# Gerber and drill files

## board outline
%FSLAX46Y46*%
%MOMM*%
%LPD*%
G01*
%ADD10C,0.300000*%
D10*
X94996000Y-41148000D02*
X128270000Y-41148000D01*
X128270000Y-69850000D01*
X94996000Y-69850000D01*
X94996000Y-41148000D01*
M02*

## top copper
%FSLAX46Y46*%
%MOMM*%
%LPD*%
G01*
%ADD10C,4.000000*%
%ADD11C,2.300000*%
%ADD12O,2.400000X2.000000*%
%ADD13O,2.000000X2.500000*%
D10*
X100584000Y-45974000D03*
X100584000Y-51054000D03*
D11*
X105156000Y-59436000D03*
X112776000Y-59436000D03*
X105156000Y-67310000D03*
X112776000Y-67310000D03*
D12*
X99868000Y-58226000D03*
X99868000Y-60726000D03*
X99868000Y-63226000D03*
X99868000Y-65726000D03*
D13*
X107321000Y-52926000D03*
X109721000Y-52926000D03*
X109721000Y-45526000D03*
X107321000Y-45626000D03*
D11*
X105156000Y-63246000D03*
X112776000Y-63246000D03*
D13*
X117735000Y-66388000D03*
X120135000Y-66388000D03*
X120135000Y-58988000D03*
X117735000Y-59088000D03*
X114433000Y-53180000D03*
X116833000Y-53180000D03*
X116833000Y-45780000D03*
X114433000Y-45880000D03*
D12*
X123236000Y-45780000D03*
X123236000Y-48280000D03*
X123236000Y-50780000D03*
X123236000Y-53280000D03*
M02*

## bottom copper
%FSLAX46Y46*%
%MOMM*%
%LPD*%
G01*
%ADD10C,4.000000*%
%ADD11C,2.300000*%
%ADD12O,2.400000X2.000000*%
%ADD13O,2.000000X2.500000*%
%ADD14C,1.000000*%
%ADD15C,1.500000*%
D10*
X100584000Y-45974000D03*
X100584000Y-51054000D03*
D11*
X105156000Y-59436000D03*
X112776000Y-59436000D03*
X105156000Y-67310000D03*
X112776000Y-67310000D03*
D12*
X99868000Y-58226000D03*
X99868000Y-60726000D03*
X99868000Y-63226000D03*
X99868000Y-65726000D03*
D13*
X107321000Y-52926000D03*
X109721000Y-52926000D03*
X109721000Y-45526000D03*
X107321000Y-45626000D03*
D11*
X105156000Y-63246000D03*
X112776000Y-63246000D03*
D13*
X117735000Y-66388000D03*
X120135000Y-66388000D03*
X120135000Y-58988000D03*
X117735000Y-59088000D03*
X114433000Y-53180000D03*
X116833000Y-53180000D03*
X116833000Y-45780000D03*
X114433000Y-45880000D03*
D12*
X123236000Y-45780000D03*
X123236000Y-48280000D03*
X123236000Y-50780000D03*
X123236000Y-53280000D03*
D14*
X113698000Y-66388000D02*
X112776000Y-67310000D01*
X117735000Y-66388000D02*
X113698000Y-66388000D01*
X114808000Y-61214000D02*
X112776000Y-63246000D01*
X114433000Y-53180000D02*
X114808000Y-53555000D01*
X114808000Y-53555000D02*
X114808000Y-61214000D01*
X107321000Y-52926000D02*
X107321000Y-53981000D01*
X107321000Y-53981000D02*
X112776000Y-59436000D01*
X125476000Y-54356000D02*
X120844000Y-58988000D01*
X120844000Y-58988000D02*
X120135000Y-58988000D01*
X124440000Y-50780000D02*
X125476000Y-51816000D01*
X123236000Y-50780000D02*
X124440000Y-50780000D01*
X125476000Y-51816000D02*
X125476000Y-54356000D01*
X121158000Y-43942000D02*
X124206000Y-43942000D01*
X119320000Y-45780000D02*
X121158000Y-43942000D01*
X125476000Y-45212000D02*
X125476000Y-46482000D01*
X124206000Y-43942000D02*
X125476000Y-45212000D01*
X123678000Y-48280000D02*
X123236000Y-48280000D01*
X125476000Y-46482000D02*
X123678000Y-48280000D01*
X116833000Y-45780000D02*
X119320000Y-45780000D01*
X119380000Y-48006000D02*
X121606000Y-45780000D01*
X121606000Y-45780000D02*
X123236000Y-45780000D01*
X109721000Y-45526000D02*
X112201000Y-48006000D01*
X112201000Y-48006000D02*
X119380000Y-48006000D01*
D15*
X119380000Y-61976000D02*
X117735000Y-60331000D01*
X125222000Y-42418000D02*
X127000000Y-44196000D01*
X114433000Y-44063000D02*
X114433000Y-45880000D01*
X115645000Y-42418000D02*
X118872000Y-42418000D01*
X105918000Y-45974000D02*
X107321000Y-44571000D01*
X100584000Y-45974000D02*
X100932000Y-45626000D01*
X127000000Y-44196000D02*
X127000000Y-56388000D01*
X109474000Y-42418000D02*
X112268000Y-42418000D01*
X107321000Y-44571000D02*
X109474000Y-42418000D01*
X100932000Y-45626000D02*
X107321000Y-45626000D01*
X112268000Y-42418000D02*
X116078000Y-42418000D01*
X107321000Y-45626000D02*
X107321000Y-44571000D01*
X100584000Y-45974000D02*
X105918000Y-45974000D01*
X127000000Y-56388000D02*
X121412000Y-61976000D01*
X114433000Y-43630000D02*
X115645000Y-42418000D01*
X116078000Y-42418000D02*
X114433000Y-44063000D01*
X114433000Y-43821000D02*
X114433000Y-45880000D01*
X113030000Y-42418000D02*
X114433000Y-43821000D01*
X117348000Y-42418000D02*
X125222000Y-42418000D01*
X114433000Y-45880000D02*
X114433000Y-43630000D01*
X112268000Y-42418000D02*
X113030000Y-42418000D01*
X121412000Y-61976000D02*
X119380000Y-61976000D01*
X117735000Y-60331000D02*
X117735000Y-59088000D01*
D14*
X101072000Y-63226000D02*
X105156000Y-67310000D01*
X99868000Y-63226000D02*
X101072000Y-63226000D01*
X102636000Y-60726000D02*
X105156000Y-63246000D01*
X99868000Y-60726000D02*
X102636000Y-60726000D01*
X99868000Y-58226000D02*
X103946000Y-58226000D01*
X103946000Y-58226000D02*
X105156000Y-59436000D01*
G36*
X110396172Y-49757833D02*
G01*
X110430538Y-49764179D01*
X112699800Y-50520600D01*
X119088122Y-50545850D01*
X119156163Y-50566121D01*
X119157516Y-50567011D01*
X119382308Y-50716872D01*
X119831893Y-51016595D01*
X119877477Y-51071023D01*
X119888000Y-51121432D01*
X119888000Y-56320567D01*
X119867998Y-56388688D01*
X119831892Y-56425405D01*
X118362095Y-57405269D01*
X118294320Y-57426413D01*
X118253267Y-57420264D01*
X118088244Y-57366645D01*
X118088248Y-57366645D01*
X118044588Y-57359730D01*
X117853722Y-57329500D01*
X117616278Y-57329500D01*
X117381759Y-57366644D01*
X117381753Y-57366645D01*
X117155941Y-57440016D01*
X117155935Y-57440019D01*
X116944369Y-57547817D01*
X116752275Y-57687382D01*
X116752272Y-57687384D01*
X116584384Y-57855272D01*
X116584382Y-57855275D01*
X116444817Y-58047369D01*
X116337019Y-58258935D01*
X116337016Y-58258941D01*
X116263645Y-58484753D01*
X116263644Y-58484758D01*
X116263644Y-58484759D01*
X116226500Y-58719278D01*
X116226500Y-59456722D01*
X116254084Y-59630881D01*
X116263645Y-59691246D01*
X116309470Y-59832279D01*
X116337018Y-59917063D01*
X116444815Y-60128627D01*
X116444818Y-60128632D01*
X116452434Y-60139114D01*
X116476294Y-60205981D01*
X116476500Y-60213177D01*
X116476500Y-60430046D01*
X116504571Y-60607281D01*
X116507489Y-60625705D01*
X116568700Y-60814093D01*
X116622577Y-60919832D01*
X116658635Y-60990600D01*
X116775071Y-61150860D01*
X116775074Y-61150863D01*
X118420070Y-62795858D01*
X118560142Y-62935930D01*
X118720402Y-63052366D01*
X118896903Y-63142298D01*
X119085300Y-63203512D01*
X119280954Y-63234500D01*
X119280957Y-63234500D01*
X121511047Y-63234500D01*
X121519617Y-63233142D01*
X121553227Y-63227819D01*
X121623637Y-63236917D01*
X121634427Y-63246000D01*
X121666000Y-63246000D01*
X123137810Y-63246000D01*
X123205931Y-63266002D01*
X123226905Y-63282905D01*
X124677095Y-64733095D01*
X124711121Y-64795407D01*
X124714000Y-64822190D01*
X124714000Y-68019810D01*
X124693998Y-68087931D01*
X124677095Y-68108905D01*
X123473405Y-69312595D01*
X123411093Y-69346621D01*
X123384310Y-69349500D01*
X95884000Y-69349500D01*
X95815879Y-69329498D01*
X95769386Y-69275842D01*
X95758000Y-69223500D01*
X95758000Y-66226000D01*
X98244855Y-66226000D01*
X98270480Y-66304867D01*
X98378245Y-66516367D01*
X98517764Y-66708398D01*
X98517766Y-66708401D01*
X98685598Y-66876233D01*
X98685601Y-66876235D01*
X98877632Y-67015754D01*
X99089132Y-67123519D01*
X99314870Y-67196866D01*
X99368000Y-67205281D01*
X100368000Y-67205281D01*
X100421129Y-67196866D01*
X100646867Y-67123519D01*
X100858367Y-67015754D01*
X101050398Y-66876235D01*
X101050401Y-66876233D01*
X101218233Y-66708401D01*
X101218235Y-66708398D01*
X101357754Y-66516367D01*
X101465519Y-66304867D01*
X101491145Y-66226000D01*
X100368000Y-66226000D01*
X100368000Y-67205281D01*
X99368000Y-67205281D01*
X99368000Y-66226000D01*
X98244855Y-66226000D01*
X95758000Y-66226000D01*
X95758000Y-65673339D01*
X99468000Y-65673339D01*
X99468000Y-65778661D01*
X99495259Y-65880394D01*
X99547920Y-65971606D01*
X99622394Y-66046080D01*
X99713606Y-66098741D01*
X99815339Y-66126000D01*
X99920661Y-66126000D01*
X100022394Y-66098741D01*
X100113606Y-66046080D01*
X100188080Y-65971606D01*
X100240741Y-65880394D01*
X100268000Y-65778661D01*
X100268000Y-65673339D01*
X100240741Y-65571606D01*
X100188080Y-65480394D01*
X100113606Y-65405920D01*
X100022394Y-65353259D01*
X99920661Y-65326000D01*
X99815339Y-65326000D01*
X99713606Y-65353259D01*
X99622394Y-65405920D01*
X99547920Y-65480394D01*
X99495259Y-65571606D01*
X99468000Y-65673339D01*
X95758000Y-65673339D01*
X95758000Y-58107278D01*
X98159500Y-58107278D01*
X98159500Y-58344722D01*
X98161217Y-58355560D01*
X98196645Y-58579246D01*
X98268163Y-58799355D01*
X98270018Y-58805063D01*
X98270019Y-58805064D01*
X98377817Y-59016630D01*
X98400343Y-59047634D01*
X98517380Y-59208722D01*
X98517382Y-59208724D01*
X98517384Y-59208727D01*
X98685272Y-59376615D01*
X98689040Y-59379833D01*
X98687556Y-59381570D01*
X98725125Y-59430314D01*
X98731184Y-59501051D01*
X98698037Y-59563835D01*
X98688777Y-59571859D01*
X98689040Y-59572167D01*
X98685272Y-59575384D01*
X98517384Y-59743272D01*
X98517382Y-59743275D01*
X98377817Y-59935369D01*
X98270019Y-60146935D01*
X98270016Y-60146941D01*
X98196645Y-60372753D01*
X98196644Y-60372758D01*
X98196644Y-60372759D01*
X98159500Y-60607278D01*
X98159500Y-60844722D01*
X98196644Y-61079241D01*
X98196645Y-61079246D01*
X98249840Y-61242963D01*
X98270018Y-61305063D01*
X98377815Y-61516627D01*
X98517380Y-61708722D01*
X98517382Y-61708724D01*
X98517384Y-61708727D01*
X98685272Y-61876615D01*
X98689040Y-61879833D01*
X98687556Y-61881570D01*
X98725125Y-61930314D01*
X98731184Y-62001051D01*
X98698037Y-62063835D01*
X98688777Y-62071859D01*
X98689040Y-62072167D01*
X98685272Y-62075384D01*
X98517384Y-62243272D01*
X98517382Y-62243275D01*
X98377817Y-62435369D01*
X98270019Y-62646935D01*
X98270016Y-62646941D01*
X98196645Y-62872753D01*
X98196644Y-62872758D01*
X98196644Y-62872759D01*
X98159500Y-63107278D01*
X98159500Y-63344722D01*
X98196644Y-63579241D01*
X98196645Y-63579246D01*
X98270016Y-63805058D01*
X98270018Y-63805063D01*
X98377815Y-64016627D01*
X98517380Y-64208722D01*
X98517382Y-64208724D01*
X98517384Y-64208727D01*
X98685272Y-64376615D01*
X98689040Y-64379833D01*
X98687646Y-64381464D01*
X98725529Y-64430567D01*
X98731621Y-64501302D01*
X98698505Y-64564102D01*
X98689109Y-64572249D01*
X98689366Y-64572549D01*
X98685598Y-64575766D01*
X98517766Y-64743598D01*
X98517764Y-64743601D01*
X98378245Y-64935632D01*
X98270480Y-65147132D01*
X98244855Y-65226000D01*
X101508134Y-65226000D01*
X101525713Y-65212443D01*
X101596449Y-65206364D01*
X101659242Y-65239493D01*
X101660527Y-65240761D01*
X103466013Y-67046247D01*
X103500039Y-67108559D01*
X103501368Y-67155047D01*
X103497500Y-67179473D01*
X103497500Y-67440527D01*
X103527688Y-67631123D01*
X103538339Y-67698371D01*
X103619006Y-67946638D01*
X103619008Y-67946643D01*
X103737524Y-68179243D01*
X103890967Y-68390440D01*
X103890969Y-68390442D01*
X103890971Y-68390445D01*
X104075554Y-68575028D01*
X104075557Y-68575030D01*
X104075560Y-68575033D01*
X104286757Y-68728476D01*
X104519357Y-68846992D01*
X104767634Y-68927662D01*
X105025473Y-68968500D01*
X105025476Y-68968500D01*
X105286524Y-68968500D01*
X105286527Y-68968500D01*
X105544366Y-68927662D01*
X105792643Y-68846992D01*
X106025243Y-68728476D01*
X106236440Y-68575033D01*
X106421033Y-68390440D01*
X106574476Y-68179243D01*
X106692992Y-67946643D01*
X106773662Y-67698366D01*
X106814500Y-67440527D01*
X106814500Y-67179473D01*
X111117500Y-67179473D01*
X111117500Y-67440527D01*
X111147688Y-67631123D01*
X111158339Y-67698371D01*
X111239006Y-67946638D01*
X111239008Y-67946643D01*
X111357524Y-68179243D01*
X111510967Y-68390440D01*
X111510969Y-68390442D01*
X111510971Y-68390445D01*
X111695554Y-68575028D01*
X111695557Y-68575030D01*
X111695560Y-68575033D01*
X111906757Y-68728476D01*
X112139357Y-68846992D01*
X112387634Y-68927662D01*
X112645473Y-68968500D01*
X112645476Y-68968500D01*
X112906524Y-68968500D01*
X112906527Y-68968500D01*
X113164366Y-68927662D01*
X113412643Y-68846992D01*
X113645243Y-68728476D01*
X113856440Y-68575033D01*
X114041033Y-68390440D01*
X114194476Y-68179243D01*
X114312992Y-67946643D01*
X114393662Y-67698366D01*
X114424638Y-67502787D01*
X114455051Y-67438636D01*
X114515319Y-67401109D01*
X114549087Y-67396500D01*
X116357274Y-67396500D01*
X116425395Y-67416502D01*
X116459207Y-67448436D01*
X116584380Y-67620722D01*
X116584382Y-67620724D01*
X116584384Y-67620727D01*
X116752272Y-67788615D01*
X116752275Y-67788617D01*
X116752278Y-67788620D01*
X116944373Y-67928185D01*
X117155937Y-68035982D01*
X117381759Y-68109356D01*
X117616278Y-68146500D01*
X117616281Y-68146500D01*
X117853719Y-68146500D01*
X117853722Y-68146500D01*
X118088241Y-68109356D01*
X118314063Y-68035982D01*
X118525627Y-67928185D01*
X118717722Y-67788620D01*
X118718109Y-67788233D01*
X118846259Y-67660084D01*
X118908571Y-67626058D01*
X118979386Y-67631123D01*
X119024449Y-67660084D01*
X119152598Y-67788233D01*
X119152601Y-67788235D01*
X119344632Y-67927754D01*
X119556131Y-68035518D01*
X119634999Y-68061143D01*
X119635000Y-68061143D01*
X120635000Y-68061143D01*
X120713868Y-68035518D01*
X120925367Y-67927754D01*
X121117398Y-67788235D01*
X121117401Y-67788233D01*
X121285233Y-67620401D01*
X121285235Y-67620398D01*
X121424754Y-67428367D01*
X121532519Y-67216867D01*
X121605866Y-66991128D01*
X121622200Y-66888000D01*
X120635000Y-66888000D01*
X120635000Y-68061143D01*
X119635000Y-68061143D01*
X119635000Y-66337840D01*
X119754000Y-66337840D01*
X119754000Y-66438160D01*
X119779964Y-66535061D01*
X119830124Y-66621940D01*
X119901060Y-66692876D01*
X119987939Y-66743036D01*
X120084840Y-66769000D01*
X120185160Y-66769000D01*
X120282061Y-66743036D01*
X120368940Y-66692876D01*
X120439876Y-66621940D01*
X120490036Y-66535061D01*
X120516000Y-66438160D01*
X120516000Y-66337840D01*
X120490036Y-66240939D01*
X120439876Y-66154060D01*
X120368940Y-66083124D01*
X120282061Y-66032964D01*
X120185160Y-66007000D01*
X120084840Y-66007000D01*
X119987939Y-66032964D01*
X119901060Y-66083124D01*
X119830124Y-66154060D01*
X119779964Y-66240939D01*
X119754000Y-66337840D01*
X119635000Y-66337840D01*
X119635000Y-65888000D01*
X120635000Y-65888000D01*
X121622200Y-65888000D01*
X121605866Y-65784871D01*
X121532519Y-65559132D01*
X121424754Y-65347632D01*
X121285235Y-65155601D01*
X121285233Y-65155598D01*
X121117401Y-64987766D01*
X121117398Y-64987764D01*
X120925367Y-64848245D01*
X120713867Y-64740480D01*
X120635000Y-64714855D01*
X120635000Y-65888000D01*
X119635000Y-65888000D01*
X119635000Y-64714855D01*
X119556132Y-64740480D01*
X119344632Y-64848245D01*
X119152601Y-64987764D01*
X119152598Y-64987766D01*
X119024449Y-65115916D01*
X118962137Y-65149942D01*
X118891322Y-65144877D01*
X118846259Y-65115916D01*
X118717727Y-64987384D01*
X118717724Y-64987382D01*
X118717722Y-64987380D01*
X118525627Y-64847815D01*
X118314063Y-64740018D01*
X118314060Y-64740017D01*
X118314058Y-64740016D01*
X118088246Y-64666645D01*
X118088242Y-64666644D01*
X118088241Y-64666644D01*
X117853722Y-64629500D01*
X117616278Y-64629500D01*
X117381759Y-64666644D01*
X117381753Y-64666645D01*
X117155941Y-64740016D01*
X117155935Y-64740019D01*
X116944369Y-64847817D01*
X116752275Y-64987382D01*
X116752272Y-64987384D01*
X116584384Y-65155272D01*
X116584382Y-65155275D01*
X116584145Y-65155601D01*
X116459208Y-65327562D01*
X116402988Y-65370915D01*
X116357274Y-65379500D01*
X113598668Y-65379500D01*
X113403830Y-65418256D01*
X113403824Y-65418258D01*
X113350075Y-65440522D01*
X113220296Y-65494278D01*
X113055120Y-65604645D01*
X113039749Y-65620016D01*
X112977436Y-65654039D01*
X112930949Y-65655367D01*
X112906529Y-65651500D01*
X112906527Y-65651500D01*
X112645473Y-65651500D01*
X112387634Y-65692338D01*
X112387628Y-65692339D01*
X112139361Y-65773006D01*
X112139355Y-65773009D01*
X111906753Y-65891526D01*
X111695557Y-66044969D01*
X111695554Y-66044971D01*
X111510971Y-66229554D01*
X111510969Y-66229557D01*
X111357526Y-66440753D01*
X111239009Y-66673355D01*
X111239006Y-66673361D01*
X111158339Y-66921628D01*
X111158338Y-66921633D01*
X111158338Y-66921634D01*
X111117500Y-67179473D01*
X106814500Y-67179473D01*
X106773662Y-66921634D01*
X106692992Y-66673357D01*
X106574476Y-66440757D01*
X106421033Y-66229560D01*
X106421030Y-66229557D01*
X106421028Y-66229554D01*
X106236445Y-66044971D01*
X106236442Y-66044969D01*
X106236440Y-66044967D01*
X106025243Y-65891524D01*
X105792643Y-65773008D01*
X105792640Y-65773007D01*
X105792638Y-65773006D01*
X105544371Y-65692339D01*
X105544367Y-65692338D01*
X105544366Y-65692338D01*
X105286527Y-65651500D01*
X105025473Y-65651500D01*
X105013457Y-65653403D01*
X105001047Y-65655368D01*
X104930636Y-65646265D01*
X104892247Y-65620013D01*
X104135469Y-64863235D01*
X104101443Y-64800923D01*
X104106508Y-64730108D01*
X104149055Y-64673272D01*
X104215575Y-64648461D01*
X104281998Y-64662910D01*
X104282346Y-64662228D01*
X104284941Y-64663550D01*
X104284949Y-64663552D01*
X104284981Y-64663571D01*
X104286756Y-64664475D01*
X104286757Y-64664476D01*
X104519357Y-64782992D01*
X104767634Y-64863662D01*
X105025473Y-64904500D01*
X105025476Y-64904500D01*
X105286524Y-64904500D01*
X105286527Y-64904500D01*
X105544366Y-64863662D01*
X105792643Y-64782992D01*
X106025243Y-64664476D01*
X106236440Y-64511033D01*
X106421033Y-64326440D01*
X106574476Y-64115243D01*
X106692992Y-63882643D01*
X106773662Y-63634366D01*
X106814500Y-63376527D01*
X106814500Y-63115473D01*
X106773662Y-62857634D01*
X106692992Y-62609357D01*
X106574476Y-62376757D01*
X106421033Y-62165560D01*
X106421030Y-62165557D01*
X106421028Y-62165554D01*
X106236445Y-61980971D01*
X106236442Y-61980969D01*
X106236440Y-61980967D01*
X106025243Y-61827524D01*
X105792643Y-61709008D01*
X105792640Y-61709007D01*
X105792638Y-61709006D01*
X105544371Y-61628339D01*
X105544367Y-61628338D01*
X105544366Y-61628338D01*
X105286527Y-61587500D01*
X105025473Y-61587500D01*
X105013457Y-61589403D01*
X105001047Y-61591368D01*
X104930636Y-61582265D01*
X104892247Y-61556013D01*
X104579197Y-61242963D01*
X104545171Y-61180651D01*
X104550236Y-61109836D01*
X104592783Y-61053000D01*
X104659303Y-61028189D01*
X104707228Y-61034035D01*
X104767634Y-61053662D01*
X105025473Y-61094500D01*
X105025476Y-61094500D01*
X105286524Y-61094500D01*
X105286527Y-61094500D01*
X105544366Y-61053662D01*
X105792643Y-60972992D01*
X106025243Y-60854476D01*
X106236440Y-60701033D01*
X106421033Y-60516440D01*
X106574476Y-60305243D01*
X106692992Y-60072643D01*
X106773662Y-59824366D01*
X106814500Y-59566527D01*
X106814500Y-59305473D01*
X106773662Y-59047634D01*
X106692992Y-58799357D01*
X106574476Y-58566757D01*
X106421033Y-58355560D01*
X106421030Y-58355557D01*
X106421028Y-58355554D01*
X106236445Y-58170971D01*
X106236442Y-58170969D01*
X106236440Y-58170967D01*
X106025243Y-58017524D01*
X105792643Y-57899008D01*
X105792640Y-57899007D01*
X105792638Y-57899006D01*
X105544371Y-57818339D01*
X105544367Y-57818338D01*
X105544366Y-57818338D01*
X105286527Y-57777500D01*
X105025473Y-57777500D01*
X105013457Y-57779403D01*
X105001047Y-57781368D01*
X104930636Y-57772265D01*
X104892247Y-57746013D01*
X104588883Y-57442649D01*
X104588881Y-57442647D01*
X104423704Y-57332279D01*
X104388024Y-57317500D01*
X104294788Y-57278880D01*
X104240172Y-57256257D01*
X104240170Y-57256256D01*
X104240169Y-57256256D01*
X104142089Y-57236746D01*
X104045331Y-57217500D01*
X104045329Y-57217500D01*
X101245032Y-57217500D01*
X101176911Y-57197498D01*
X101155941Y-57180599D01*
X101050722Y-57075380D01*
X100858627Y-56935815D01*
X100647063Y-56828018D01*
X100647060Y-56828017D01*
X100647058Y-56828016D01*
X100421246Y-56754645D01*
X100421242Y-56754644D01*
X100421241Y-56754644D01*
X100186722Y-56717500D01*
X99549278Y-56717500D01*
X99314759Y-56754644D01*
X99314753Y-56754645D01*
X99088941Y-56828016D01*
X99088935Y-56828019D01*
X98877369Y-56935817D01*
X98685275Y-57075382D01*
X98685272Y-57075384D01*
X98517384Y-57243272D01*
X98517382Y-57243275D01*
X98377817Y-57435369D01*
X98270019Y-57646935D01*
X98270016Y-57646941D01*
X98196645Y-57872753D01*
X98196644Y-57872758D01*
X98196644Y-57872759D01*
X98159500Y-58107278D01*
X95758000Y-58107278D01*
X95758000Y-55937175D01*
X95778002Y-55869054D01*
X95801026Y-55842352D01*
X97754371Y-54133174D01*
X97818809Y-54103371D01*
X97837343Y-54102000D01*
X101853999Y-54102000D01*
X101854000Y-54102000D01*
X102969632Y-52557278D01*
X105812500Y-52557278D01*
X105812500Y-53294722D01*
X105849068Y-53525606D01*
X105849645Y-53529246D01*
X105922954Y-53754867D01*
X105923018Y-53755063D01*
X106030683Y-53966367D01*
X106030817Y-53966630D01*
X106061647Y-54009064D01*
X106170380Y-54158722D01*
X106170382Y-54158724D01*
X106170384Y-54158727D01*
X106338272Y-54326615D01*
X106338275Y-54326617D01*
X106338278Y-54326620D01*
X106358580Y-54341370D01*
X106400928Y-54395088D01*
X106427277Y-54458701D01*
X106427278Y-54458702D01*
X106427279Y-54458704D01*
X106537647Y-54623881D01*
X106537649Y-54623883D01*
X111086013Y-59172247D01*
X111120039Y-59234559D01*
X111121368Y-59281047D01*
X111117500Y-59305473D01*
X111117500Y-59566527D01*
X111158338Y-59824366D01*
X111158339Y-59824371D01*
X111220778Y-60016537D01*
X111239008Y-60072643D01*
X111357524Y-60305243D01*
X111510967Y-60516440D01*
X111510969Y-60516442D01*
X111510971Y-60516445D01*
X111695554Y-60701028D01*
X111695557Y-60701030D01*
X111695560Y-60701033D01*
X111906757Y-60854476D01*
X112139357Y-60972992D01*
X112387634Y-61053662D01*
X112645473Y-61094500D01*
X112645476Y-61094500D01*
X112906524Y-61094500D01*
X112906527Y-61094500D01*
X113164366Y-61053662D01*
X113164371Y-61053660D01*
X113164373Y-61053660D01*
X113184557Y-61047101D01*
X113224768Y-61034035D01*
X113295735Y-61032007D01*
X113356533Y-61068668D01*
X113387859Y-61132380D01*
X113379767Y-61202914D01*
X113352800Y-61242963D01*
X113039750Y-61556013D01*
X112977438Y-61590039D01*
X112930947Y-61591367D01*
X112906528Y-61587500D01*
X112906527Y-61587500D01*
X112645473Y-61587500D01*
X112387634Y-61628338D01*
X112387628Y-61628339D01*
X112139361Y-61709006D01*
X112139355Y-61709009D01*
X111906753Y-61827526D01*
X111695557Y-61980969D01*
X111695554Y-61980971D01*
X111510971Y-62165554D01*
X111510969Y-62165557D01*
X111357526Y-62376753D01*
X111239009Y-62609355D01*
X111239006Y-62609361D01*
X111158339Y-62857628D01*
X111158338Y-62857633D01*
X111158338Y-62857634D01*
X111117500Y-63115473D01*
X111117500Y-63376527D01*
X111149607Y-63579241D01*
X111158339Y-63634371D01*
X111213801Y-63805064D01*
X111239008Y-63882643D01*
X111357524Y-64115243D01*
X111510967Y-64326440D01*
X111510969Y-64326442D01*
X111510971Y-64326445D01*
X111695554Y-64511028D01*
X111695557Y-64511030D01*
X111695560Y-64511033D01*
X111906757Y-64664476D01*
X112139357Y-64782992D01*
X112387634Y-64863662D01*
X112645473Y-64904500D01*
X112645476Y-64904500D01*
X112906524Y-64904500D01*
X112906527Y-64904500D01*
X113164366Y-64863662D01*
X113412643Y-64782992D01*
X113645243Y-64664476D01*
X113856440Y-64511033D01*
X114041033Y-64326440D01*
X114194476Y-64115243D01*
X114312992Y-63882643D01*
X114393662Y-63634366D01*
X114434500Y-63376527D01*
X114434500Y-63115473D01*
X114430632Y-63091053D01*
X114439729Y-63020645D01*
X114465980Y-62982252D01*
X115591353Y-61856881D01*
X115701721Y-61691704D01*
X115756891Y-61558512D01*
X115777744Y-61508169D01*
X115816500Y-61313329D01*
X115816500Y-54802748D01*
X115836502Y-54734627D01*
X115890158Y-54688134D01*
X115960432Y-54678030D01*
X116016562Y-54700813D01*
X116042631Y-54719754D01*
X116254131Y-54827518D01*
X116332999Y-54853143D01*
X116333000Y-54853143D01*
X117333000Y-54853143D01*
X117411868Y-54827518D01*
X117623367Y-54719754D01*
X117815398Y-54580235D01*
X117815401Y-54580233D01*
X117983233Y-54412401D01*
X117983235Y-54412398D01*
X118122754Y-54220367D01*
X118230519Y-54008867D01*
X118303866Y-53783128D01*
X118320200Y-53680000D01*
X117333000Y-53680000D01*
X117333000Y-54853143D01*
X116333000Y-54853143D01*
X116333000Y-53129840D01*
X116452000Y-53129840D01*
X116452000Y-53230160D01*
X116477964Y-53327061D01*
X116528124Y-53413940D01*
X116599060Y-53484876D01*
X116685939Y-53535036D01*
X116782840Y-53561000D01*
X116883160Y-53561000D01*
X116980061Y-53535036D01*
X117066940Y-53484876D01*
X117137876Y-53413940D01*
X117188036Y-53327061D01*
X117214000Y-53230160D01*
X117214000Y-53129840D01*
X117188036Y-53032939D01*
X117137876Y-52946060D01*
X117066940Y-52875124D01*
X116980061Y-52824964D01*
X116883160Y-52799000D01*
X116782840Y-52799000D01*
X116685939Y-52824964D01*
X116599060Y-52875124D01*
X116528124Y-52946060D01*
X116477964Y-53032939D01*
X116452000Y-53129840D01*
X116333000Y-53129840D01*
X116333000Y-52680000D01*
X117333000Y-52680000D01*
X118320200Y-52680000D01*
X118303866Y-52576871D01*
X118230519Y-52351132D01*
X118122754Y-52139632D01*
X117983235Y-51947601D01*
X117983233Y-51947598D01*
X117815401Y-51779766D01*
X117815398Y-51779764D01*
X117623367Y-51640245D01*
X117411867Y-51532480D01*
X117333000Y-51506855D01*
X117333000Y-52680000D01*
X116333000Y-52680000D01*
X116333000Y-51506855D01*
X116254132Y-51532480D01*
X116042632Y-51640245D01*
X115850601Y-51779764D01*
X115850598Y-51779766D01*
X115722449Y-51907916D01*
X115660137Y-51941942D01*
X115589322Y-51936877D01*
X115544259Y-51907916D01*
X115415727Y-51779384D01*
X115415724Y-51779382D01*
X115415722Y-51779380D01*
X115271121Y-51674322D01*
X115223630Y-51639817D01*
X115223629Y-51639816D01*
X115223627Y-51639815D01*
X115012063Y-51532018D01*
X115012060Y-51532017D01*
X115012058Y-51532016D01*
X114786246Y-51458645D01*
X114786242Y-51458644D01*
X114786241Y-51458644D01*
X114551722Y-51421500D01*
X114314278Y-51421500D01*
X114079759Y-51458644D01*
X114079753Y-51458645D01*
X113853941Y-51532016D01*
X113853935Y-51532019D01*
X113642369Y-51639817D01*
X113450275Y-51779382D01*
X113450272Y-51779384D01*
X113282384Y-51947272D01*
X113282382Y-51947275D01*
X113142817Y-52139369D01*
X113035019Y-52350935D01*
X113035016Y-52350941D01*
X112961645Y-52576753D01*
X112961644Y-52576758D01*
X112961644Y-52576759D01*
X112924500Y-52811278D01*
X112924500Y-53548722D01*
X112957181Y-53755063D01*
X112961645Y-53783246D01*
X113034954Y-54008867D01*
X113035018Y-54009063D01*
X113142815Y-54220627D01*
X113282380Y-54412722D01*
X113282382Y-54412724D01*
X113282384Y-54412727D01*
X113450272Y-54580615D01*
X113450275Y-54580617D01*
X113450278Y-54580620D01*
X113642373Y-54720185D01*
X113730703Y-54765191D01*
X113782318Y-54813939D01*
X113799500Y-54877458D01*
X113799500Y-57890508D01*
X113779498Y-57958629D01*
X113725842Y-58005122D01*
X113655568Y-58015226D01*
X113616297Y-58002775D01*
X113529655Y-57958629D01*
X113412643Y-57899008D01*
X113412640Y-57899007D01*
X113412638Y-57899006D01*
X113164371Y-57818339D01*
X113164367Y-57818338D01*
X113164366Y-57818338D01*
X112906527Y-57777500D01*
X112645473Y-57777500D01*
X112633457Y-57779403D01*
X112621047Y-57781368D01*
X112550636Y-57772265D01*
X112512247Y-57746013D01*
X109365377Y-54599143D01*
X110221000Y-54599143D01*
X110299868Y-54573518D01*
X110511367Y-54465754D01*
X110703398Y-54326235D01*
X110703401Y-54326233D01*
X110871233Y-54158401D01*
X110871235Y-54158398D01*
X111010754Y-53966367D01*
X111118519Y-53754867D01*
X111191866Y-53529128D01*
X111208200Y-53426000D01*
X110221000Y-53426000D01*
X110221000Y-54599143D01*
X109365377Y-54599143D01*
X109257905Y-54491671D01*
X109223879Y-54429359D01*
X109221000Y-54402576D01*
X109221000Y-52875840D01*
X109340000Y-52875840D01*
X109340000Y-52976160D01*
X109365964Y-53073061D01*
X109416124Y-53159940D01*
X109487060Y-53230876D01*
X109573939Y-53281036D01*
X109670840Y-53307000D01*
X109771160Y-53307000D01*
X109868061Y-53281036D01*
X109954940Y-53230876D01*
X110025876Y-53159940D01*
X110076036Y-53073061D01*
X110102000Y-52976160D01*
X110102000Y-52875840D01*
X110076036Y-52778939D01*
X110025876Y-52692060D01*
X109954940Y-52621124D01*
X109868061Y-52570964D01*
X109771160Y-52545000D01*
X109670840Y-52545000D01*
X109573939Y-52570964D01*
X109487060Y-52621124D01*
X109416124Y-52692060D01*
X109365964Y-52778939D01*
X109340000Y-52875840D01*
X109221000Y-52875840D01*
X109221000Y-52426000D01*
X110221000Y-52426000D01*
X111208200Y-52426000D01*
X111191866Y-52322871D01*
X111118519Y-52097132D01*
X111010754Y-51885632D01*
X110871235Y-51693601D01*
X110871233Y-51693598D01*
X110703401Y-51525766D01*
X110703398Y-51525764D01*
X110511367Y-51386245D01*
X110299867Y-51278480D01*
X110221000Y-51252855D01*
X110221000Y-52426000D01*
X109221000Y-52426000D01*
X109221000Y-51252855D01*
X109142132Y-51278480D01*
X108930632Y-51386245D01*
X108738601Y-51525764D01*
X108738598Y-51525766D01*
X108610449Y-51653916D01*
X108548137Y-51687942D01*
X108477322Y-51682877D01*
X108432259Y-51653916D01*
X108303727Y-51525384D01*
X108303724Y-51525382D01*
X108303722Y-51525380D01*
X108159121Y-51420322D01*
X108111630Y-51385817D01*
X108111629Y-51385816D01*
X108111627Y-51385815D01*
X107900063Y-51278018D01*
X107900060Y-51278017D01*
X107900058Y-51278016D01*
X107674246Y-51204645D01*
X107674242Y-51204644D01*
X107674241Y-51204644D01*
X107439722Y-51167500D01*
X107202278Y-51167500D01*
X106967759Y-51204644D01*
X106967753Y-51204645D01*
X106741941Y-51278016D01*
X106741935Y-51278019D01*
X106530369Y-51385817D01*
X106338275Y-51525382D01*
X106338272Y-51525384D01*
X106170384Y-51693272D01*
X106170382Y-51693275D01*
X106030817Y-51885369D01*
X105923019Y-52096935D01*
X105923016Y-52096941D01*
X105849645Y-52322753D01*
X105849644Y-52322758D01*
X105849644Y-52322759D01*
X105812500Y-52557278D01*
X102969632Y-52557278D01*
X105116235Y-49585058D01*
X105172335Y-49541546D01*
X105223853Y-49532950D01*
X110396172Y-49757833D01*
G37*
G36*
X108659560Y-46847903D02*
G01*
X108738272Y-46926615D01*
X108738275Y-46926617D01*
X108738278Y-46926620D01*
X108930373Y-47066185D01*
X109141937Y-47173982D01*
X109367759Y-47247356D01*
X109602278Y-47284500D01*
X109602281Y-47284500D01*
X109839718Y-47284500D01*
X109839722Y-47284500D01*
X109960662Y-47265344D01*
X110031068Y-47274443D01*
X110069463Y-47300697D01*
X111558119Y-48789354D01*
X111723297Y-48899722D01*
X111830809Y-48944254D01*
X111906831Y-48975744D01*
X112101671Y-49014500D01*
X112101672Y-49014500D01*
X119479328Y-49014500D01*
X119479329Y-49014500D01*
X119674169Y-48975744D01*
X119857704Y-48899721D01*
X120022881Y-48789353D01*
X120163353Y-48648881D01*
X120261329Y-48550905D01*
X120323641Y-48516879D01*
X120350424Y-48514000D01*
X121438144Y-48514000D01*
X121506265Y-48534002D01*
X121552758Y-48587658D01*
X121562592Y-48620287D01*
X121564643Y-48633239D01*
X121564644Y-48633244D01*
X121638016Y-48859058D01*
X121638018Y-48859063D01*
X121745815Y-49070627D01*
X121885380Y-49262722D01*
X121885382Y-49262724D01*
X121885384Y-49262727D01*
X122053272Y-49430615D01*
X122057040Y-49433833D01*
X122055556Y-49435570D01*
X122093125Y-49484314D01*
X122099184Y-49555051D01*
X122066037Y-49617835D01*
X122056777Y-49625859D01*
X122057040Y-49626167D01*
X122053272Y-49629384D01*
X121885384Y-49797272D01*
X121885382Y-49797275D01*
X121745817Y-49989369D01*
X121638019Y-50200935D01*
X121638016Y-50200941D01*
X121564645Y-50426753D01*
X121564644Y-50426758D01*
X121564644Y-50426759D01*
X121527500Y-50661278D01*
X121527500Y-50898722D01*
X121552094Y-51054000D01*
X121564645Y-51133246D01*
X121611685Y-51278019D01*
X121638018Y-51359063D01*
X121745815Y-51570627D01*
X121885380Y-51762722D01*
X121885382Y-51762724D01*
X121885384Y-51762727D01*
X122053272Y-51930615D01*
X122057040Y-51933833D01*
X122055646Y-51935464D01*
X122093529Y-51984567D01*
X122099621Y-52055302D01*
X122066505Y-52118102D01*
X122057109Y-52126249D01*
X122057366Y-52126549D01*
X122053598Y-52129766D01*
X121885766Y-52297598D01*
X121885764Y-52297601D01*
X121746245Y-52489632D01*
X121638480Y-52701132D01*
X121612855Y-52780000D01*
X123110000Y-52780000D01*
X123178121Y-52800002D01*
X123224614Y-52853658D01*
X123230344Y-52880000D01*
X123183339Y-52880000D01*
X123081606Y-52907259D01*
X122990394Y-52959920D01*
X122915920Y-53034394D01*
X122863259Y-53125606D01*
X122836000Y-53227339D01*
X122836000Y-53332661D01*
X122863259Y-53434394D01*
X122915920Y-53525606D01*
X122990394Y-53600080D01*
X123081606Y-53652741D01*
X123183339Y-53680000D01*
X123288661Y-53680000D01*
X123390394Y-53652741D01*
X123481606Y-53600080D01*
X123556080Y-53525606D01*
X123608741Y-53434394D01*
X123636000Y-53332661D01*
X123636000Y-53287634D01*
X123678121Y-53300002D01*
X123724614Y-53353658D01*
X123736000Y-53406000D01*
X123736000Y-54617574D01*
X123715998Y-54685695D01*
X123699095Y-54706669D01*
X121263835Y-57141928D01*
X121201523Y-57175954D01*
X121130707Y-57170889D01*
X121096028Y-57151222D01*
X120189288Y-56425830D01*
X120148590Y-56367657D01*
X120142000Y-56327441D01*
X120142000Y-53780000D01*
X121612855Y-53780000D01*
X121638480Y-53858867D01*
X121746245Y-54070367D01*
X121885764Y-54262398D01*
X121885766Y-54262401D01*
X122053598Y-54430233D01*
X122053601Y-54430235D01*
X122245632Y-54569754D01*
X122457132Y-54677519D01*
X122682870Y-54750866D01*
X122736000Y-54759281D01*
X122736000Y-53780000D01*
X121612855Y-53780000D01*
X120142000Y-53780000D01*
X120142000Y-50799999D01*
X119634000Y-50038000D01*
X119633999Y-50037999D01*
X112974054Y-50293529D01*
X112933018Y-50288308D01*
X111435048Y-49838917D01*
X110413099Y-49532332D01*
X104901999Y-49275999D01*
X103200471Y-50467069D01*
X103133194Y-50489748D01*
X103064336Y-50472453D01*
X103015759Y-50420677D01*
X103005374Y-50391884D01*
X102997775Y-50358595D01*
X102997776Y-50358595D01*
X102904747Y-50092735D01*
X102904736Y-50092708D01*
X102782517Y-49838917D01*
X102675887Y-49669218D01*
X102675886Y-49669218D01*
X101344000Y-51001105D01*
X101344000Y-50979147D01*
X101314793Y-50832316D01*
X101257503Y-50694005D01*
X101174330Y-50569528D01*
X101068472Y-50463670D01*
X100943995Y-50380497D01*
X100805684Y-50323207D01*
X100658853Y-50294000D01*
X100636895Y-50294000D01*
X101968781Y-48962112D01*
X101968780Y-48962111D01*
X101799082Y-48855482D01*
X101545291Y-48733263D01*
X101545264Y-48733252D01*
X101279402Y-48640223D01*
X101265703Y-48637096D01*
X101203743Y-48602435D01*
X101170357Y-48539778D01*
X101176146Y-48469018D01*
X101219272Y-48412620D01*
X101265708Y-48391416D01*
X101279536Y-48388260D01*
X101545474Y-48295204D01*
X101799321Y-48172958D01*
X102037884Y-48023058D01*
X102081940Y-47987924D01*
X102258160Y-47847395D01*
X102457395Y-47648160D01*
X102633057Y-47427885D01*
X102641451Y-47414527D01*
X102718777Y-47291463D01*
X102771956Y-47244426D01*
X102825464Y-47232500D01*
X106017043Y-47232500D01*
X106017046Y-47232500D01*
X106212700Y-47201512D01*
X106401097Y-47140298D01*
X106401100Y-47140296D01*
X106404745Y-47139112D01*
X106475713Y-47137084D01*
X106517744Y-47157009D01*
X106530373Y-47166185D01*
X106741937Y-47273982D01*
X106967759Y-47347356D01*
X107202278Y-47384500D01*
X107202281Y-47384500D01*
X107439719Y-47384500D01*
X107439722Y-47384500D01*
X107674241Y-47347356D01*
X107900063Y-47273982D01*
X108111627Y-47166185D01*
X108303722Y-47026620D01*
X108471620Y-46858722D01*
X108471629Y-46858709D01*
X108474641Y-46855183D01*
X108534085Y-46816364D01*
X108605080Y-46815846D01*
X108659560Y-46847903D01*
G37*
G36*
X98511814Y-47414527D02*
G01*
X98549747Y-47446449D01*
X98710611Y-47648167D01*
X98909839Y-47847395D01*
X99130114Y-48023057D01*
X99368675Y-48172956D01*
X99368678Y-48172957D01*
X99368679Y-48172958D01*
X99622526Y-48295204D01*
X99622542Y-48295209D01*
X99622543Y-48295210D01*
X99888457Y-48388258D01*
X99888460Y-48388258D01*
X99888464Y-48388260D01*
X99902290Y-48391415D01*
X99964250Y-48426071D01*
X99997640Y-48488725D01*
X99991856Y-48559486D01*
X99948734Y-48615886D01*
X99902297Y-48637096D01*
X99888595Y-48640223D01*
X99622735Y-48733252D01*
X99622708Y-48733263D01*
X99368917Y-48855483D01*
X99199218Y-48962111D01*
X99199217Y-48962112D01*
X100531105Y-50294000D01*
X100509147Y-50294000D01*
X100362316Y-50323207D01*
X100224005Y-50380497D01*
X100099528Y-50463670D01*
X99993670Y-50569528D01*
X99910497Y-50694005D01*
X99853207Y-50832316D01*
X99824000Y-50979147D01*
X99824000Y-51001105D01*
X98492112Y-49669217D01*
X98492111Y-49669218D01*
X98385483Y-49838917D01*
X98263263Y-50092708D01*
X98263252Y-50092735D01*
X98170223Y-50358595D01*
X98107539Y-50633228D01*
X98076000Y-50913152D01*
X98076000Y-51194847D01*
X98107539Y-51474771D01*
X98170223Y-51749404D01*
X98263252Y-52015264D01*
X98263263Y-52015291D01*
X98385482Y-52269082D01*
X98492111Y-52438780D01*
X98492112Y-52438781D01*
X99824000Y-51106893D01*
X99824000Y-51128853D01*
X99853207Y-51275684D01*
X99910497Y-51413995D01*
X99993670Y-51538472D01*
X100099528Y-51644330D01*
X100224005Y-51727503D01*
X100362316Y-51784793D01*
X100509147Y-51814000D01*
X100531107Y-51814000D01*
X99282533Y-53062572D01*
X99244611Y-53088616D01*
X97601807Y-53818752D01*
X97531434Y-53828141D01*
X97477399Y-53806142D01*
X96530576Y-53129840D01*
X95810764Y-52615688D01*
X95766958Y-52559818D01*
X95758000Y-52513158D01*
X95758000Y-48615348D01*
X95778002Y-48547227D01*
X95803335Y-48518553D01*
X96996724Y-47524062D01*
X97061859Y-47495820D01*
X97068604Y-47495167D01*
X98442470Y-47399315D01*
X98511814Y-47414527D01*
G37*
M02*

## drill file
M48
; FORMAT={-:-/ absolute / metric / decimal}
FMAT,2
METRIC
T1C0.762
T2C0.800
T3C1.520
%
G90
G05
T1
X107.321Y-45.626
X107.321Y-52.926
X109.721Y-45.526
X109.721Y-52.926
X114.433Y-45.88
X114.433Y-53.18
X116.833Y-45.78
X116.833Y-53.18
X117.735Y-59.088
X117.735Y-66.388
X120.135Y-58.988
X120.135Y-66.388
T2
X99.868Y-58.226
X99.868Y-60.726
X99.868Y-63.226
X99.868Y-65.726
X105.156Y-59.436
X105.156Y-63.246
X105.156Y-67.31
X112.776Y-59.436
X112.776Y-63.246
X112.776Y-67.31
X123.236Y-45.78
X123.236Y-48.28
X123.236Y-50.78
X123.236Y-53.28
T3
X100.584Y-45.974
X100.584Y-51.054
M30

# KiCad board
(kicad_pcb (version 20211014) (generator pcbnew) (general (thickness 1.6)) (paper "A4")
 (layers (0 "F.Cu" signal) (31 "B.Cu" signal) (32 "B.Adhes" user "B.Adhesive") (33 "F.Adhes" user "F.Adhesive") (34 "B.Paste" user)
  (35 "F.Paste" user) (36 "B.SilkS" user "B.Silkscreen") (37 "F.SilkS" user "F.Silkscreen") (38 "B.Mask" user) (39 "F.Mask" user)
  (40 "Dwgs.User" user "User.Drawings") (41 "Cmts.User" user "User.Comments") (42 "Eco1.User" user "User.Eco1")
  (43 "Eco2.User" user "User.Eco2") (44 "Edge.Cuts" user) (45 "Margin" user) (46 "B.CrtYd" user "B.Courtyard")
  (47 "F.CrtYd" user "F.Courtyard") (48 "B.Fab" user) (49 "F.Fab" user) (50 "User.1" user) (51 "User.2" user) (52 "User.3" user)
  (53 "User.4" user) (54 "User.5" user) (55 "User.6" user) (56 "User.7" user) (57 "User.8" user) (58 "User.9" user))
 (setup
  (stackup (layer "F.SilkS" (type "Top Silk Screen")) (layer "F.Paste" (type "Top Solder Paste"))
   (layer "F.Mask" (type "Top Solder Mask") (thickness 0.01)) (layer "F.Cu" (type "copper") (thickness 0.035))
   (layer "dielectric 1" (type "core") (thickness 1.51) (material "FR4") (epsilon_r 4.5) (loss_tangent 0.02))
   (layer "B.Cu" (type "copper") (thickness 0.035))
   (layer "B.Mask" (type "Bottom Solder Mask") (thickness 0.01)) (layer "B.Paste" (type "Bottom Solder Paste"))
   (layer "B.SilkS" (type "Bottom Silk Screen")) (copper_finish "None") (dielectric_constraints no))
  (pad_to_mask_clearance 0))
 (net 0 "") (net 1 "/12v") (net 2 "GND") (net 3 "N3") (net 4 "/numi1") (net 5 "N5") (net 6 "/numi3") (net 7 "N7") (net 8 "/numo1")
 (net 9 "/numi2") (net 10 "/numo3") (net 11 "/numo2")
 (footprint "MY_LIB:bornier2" (layer "F.Cu") (at 100.584 45.974 -90)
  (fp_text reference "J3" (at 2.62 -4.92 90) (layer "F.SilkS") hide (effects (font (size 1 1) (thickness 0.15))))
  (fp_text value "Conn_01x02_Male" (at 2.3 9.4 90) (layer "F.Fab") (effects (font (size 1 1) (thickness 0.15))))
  (pad "1" thru_hole circle locked (at 0 0 270) (size 4 4) (drill 1.52) (layers *.Cu *.Mask) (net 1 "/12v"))
  (pad "2" thru_hole circle locked (at 5.08 0 270) (size 4 4) (drill 1.52) (layers *.Cu *.Mask) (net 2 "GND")))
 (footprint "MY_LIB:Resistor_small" (layer "F.Cu") (at 105.156 59.436)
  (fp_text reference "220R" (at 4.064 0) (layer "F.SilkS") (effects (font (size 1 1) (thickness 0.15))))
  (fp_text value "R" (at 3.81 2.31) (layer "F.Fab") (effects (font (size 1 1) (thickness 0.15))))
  (pad "1" thru_hole circle locked (at 0 0) (size 2.3 2.3) (drill 0.8) (layers *.Cu *.Mask) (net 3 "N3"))
  (pad "2" thru_hole circle locked (at 7.62 0) (size 2.3 2.3) (drill 0.8) (layers *.Cu *.Mask) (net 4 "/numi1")))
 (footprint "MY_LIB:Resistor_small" (layer "F.Cu") (at 105.156 67.31)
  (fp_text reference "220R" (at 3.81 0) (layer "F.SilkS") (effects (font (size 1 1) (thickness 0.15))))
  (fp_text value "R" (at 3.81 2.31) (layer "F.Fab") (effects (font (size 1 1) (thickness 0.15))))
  (pad "1" thru_hole circle locked (at 0 0) (size 2.3 2.3) (drill 0.8) (layers *.Cu *.Mask) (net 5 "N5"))
  (pad "2" thru_hole circle locked (at 7.62 0) (size 2.3 2.3) (drill 0.8) (layers *.Cu *.Mask) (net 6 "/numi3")))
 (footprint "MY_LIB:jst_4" (layer "F.Cu") (at 99.868 58.226 -90)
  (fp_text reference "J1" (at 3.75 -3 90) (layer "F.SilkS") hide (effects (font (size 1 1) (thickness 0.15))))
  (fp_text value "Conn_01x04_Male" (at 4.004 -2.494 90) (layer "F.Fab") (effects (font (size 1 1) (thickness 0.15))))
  (pad "1" thru_hole oval locked (at 0 0 270) (size 2 2.4) (drill 0.8) (layers *.Cu *.Mask) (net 3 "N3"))
  (pad "2" thru_hole oval locked (at 2.5 0 270) (size 2 2.4) (drill 0.8) (layers *.Cu *.Mask) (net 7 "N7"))
  (pad "3" thru_hole oval locked (at 5 0 270) (size 2 2.4) (drill 0.8) (layers *.Cu *.Mask) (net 5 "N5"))
  (pad "4" thru_hole oval locked (at 7.5 0 270) (size 2 2.4) (drill 0.8) (layers *.Cu *.Mask) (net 2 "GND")))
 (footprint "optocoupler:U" (layer "F.Cu") (at 112.121 50.026 90)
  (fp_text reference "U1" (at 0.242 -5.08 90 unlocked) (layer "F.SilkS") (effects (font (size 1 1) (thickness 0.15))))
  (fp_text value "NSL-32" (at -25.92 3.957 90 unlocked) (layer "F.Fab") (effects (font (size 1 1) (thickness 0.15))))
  (pad "1" thru_hole oval (at -2.9 -4.8 90) (size 2.5 2) (drill 0.762) (layers *.Cu *.Mask) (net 4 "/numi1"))
  (pad "2" thru_hole oval (at -2.9 -2.4 90) (size 2.5 2) (drill 0.762) (layers *.Cu *.Mask) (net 2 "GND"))
  (pad "3" thru_hole oval (at 4.5 -2.4 90) (size 2.5 2) (drill 0.762) (layers *.Cu *.Mask) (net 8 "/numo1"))
  (pad "4" thru_hole oval (at 4.4 -4.8 90) (size 2.5 2) (drill 0.762) (layers *.Cu *.Mask) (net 1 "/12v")))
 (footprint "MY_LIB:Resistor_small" (layer "F.Cu") (at 105.156 63.246)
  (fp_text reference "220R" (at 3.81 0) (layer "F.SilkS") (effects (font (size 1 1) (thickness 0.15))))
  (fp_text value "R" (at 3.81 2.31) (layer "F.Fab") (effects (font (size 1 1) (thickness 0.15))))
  (pad "1" thru_hole circle locked (at 0 0) (size 2.3 2.3) (drill 0.8) (layers *.Cu *.Mask) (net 7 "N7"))
  (pad "2" thru_hole circle locked (at 7.62 0) (size 2.3 2.3) (drill 0.8) (layers *.Cu *.Mask) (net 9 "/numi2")))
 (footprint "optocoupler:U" (layer "F.Cu") (at 122.535 63.488 90)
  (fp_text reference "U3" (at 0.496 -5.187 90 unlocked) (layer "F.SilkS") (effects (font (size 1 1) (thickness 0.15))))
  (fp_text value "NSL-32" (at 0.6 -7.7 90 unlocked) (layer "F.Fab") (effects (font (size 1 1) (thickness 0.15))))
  (pad "1" thru_hole oval (at -2.9 -4.8 90) (size 2.5 2) (drill 0.762) (layers *.Cu *.Mask) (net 6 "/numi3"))
  (pad "2" thru_hole oval (at -2.9 -2.4 90) (size 2.5 2) (drill 0.762) (layers *.Cu *.Mask) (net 2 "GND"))
  (pad "3" thru_hole oval (at 4.5 -2.4 90) (size 2.5 2) (drill 0.762) (layers *.Cu *.Mask) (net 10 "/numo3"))
  (pad "4" thru_hole oval (at 4.4 -4.8 90) (size 2.5 2) (drill 0.762) (layers *.Cu *.Mask) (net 1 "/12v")))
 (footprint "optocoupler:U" (layer "F.Cu") (at 119.233 50.28 90)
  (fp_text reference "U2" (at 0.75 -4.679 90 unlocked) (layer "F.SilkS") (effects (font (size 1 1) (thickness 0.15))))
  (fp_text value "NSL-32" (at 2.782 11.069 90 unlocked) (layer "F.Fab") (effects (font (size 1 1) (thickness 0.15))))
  (pad "1" thru_hole oval (at -2.9 -4.8 90) (size 2.5 2) (drill 0.762) (layers *.Cu *.Mask) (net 9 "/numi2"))
  (pad "2" thru_hole oval (at -2.9 -2.4 90) (size 2.5 2) (drill 0.762) (layers *.Cu *.Mask) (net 2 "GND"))
  (pad "3" thru_hole oval (at 4.5 -2.4 90) (size 2.5 2) (drill 0.762) (layers *.Cu *.Mask) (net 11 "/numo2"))
  (pad "4" thru_hole oval (at 4.4 -4.8 90) (size 2.5 2) (drill 0.762) (layers *.Cu *.Mask) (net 1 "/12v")))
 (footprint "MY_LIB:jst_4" (layer "F.Cu") (at 123.236 45.78 -90)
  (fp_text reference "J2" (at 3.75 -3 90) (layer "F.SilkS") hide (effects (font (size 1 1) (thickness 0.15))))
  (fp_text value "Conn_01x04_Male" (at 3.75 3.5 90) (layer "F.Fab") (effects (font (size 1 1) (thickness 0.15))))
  (pad "1" thru_hole oval locked (at 0 0 270) (size 2 2.4) (drill 0.8) (layers *.Cu *.Mask) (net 8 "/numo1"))
  (pad "2" thru_hole oval locked (at 2.5 0 270) (size 2 2.4) (drill 0.8) (layers *.Cu *.Mask) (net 11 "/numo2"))
  (pad "3" thru_hole oval locked (at 5 0 270) (size 2 2.4) (drill 0.8) (layers *.Cu *.Mask) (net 10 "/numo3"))
  (pad "4" thru_hole oval locked (at 7.5 0 270) (size 2 2.4) (drill 0.8) (layers *.Cu *.Mask) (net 2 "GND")))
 (gr_rect (start 94.996 41.148) (end 128.27 69.85) (layer "Edge.Cuts") (width 0.3) (fill none))
 (segment (start 113.698 66.388) (end 112.776 67.31) (width 1) (layer "B.Cu") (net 6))
 (segment (start 117.735 66.388) (end 113.698 66.388) (width 1) (layer "B.Cu") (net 6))
 (segment (start 114.808 61.214) (end 112.776 63.246) (width 1) (layer "B.Cu") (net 9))
 (segment (start 114.433 53.18) (end 114.808 53.555) (width 1) (layer "B.Cu") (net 9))
 (segment (start 114.808 53.555) (end 114.808 61.214) (width 1) (layer "B.Cu") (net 9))
 (segment (start 107.321 52.926) (end 107.321 53.981) (width 1) (layer "B.Cu") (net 4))
 (segment (start 107.321 53.981) (end 112.776 59.436) (width 1) (layer "B.Cu") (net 4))
 (segment (start 125.476 54.356) (end 120.844 58.988) (width 1) (layer "B.Cu") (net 10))
 (segment (start 120.844 58.988) (end 120.135 58.988) (width 1) (layer "B.Cu") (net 10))
 (segment (start 124.44 50.78) (end 125.476 51.816) (width 1) (layer "B.Cu") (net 10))
 (segment (start 123.236 50.78) (end 124.44 50.78) (width 1) (layer "B.Cu") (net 10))
 (segment (start 125.476 51.816) (end 125.476 54.356) (width 1) (layer "B.Cu") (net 10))
 (segment (start 121.158 43.942) (end 124.206 43.942) (width 1) (layer "B.Cu") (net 11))
 (segment (start 119.32 45.78) (end 121.158 43.942) (width 1) (layer "B.Cu") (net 11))
 (segment (start 125.476 45.212) (end 125.476 46.482) (width 1) (layer "B.Cu") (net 11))
 (segment (start 124.206 43.942) (end 125.476 45.212) (width 1) (layer "B.Cu") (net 11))
 (segment (start 123.678 48.28) (end 123.236 48.28) (width 1) (layer "B.Cu") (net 11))
 (segment (start 125.476 46.482) (end 123.678 48.28) (width 1) (layer "B.Cu") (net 11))
 (segment (start 116.833 45.78) (end 119.32 45.78) (width 1) (layer "B.Cu") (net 11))
 (segment (start 119.38 48.006) (end 121.606 45.78) (width 1) (layer "B.Cu") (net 8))
 (segment (start 121.606 45.78) (end 123.236 45.78) (width 1) (layer "B.Cu") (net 8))
 (segment (start 109.721 45.526) (end 112.201 48.006) (width 1) (layer "B.Cu") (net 8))
 (segment (start 112.201 48.006) (end 119.38 48.006) (width 1) (layer "B.Cu") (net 8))
 (segment (start 119.38 61.976) (end 117.735 60.331) (width 1.5) (layer "B.Cu") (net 1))
 (segment (start 125.222 42.418) (end 127 44.196) (width 1.5) (layer "B.Cu") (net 1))
 (segment (start 114.433 44.063) (end 114.433 45.88) (width 1.5) (layer "B.Cu") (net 1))
 (segment (start 115.645 42.418) (end 118.872 42.418) (width 1.5) (layer "B.Cu") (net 1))
 (segment (start 105.918 45.974) (end 107.321 44.571) (width 1.5) (layer "B.Cu") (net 1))
 (segment (start 100.584 45.974) (end 100.932 45.626) (width 1.5) (layer "B.Cu") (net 1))
 (segment (start 127 44.196) (end 127 56.388) (width 1.5) (layer "B.Cu") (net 1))
 (segment (start 109.474 42.418) (end 112.268 42.418) (width 1.5) (layer "B.Cu") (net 1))
 (segment (start 107.321 44.571) (end 109.474 42.418) (width 1.5) (layer "B.Cu") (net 1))
 (segment (start 100.932 45.626) (end 107.321 45.626) (width 1.5) (layer "B.Cu") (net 1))
 (segment (start 112.268 42.418) (end 116.078 42.418) (width 1.5) (layer "B.Cu") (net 1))
 (segment (start 107.321 45.626) (end 107.321 44.571) (width 1.5) (layer "B.Cu") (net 1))
 (segment (start 100.584 45.974) (end 105.918 45.974) (width 1.5) (layer "B.Cu") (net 1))
 (segment (start 127 56.388) (end 121.412 61.976) (width 1.5) (layer "B.Cu") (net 1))
 (segment (start 114.433 43.63) (end 115.645 42.418) (width 1.5) (layer "B.Cu") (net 1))
 (segment (start 116.078 42.418) (end 114.433 44.063) (width 1.5) (layer "B.Cu") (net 1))
 (segment (start 114.433 43.821) (end 114.433 45.88) (width 1.5) (layer "B.Cu") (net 1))
 (segment (start 113.03 42.418) (end 114.433 43.821) (width 1.5) (layer "B.Cu") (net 1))
 (segment (start 117.348 42.418) (end 125.222 42.418) (width 1.5) (layer "B.Cu") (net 1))
 (segment (start 114.433 45.88) (end 114.433 43.63) (width 1.5) (layer "B.Cu") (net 1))
 (segment (start 112.268 42.418) (end 113.03 42.418) (width 1.5) (layer "B.Cu") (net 1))
 (segment (start 121.412 61.976) (end 119.38 61.976) (width 1.5) (layer "B.Cu") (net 1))
 (segment (start 117.735 60.331) (end 117.735 59.088) (width 1.5) (layer "B.Cu") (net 1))
 (segment (start 101.072 63.226) (end 105.156 67.31) (width 1) (layer "B.Cu") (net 5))
 (segment (start 99.868 63.226) (end 101.072 63.226) (width 1) (layer "B.Cu") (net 5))
 (segment (start 102.636 60.726) (end 105.156 63.246) (width 1) (layer "B.Cu") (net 7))
 (segment (start 99.868 60.726) (end 102.636 60.726) (width 1) (layer "B.Cu") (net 7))
 (segment (start 99.868 58.226) (end 103.946 58.226) (width 1) (layer "B.Cu") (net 3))
 (segment (start 103.946 58.226) (end 105.156 59.436) (width 1) (layer "B.Cu") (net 3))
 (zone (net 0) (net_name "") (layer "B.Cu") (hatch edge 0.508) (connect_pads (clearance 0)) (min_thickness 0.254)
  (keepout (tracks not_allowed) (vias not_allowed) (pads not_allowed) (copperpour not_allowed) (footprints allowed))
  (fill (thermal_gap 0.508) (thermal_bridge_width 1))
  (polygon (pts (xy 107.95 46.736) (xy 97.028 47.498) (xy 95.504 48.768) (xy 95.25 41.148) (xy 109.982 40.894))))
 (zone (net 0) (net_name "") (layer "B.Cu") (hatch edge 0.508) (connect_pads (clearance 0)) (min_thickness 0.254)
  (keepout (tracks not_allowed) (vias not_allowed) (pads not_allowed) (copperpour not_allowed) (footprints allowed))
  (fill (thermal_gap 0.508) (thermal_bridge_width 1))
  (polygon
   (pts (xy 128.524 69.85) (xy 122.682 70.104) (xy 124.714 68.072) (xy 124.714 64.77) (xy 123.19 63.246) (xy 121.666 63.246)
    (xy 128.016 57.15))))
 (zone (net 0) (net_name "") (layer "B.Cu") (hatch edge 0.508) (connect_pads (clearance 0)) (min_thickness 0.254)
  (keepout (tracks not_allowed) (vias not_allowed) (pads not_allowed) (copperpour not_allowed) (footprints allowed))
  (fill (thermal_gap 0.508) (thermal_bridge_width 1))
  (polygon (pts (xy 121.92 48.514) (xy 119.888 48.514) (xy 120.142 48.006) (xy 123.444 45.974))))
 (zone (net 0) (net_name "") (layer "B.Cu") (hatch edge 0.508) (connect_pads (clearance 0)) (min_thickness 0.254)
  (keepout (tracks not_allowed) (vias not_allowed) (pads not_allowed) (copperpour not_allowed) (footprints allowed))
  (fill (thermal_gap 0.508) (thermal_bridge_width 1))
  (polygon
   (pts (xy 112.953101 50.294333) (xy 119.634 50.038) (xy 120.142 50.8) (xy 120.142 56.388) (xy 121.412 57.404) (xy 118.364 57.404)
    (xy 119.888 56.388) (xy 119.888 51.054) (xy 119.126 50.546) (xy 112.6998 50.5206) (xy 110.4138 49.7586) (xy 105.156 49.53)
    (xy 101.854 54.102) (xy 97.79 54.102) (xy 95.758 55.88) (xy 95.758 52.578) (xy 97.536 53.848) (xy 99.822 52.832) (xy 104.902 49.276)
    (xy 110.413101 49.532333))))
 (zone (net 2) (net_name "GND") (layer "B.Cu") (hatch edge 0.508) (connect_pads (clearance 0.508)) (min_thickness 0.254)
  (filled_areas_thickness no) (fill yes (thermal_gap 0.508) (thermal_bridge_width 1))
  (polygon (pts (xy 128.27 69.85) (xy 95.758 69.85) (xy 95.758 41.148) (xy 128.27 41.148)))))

